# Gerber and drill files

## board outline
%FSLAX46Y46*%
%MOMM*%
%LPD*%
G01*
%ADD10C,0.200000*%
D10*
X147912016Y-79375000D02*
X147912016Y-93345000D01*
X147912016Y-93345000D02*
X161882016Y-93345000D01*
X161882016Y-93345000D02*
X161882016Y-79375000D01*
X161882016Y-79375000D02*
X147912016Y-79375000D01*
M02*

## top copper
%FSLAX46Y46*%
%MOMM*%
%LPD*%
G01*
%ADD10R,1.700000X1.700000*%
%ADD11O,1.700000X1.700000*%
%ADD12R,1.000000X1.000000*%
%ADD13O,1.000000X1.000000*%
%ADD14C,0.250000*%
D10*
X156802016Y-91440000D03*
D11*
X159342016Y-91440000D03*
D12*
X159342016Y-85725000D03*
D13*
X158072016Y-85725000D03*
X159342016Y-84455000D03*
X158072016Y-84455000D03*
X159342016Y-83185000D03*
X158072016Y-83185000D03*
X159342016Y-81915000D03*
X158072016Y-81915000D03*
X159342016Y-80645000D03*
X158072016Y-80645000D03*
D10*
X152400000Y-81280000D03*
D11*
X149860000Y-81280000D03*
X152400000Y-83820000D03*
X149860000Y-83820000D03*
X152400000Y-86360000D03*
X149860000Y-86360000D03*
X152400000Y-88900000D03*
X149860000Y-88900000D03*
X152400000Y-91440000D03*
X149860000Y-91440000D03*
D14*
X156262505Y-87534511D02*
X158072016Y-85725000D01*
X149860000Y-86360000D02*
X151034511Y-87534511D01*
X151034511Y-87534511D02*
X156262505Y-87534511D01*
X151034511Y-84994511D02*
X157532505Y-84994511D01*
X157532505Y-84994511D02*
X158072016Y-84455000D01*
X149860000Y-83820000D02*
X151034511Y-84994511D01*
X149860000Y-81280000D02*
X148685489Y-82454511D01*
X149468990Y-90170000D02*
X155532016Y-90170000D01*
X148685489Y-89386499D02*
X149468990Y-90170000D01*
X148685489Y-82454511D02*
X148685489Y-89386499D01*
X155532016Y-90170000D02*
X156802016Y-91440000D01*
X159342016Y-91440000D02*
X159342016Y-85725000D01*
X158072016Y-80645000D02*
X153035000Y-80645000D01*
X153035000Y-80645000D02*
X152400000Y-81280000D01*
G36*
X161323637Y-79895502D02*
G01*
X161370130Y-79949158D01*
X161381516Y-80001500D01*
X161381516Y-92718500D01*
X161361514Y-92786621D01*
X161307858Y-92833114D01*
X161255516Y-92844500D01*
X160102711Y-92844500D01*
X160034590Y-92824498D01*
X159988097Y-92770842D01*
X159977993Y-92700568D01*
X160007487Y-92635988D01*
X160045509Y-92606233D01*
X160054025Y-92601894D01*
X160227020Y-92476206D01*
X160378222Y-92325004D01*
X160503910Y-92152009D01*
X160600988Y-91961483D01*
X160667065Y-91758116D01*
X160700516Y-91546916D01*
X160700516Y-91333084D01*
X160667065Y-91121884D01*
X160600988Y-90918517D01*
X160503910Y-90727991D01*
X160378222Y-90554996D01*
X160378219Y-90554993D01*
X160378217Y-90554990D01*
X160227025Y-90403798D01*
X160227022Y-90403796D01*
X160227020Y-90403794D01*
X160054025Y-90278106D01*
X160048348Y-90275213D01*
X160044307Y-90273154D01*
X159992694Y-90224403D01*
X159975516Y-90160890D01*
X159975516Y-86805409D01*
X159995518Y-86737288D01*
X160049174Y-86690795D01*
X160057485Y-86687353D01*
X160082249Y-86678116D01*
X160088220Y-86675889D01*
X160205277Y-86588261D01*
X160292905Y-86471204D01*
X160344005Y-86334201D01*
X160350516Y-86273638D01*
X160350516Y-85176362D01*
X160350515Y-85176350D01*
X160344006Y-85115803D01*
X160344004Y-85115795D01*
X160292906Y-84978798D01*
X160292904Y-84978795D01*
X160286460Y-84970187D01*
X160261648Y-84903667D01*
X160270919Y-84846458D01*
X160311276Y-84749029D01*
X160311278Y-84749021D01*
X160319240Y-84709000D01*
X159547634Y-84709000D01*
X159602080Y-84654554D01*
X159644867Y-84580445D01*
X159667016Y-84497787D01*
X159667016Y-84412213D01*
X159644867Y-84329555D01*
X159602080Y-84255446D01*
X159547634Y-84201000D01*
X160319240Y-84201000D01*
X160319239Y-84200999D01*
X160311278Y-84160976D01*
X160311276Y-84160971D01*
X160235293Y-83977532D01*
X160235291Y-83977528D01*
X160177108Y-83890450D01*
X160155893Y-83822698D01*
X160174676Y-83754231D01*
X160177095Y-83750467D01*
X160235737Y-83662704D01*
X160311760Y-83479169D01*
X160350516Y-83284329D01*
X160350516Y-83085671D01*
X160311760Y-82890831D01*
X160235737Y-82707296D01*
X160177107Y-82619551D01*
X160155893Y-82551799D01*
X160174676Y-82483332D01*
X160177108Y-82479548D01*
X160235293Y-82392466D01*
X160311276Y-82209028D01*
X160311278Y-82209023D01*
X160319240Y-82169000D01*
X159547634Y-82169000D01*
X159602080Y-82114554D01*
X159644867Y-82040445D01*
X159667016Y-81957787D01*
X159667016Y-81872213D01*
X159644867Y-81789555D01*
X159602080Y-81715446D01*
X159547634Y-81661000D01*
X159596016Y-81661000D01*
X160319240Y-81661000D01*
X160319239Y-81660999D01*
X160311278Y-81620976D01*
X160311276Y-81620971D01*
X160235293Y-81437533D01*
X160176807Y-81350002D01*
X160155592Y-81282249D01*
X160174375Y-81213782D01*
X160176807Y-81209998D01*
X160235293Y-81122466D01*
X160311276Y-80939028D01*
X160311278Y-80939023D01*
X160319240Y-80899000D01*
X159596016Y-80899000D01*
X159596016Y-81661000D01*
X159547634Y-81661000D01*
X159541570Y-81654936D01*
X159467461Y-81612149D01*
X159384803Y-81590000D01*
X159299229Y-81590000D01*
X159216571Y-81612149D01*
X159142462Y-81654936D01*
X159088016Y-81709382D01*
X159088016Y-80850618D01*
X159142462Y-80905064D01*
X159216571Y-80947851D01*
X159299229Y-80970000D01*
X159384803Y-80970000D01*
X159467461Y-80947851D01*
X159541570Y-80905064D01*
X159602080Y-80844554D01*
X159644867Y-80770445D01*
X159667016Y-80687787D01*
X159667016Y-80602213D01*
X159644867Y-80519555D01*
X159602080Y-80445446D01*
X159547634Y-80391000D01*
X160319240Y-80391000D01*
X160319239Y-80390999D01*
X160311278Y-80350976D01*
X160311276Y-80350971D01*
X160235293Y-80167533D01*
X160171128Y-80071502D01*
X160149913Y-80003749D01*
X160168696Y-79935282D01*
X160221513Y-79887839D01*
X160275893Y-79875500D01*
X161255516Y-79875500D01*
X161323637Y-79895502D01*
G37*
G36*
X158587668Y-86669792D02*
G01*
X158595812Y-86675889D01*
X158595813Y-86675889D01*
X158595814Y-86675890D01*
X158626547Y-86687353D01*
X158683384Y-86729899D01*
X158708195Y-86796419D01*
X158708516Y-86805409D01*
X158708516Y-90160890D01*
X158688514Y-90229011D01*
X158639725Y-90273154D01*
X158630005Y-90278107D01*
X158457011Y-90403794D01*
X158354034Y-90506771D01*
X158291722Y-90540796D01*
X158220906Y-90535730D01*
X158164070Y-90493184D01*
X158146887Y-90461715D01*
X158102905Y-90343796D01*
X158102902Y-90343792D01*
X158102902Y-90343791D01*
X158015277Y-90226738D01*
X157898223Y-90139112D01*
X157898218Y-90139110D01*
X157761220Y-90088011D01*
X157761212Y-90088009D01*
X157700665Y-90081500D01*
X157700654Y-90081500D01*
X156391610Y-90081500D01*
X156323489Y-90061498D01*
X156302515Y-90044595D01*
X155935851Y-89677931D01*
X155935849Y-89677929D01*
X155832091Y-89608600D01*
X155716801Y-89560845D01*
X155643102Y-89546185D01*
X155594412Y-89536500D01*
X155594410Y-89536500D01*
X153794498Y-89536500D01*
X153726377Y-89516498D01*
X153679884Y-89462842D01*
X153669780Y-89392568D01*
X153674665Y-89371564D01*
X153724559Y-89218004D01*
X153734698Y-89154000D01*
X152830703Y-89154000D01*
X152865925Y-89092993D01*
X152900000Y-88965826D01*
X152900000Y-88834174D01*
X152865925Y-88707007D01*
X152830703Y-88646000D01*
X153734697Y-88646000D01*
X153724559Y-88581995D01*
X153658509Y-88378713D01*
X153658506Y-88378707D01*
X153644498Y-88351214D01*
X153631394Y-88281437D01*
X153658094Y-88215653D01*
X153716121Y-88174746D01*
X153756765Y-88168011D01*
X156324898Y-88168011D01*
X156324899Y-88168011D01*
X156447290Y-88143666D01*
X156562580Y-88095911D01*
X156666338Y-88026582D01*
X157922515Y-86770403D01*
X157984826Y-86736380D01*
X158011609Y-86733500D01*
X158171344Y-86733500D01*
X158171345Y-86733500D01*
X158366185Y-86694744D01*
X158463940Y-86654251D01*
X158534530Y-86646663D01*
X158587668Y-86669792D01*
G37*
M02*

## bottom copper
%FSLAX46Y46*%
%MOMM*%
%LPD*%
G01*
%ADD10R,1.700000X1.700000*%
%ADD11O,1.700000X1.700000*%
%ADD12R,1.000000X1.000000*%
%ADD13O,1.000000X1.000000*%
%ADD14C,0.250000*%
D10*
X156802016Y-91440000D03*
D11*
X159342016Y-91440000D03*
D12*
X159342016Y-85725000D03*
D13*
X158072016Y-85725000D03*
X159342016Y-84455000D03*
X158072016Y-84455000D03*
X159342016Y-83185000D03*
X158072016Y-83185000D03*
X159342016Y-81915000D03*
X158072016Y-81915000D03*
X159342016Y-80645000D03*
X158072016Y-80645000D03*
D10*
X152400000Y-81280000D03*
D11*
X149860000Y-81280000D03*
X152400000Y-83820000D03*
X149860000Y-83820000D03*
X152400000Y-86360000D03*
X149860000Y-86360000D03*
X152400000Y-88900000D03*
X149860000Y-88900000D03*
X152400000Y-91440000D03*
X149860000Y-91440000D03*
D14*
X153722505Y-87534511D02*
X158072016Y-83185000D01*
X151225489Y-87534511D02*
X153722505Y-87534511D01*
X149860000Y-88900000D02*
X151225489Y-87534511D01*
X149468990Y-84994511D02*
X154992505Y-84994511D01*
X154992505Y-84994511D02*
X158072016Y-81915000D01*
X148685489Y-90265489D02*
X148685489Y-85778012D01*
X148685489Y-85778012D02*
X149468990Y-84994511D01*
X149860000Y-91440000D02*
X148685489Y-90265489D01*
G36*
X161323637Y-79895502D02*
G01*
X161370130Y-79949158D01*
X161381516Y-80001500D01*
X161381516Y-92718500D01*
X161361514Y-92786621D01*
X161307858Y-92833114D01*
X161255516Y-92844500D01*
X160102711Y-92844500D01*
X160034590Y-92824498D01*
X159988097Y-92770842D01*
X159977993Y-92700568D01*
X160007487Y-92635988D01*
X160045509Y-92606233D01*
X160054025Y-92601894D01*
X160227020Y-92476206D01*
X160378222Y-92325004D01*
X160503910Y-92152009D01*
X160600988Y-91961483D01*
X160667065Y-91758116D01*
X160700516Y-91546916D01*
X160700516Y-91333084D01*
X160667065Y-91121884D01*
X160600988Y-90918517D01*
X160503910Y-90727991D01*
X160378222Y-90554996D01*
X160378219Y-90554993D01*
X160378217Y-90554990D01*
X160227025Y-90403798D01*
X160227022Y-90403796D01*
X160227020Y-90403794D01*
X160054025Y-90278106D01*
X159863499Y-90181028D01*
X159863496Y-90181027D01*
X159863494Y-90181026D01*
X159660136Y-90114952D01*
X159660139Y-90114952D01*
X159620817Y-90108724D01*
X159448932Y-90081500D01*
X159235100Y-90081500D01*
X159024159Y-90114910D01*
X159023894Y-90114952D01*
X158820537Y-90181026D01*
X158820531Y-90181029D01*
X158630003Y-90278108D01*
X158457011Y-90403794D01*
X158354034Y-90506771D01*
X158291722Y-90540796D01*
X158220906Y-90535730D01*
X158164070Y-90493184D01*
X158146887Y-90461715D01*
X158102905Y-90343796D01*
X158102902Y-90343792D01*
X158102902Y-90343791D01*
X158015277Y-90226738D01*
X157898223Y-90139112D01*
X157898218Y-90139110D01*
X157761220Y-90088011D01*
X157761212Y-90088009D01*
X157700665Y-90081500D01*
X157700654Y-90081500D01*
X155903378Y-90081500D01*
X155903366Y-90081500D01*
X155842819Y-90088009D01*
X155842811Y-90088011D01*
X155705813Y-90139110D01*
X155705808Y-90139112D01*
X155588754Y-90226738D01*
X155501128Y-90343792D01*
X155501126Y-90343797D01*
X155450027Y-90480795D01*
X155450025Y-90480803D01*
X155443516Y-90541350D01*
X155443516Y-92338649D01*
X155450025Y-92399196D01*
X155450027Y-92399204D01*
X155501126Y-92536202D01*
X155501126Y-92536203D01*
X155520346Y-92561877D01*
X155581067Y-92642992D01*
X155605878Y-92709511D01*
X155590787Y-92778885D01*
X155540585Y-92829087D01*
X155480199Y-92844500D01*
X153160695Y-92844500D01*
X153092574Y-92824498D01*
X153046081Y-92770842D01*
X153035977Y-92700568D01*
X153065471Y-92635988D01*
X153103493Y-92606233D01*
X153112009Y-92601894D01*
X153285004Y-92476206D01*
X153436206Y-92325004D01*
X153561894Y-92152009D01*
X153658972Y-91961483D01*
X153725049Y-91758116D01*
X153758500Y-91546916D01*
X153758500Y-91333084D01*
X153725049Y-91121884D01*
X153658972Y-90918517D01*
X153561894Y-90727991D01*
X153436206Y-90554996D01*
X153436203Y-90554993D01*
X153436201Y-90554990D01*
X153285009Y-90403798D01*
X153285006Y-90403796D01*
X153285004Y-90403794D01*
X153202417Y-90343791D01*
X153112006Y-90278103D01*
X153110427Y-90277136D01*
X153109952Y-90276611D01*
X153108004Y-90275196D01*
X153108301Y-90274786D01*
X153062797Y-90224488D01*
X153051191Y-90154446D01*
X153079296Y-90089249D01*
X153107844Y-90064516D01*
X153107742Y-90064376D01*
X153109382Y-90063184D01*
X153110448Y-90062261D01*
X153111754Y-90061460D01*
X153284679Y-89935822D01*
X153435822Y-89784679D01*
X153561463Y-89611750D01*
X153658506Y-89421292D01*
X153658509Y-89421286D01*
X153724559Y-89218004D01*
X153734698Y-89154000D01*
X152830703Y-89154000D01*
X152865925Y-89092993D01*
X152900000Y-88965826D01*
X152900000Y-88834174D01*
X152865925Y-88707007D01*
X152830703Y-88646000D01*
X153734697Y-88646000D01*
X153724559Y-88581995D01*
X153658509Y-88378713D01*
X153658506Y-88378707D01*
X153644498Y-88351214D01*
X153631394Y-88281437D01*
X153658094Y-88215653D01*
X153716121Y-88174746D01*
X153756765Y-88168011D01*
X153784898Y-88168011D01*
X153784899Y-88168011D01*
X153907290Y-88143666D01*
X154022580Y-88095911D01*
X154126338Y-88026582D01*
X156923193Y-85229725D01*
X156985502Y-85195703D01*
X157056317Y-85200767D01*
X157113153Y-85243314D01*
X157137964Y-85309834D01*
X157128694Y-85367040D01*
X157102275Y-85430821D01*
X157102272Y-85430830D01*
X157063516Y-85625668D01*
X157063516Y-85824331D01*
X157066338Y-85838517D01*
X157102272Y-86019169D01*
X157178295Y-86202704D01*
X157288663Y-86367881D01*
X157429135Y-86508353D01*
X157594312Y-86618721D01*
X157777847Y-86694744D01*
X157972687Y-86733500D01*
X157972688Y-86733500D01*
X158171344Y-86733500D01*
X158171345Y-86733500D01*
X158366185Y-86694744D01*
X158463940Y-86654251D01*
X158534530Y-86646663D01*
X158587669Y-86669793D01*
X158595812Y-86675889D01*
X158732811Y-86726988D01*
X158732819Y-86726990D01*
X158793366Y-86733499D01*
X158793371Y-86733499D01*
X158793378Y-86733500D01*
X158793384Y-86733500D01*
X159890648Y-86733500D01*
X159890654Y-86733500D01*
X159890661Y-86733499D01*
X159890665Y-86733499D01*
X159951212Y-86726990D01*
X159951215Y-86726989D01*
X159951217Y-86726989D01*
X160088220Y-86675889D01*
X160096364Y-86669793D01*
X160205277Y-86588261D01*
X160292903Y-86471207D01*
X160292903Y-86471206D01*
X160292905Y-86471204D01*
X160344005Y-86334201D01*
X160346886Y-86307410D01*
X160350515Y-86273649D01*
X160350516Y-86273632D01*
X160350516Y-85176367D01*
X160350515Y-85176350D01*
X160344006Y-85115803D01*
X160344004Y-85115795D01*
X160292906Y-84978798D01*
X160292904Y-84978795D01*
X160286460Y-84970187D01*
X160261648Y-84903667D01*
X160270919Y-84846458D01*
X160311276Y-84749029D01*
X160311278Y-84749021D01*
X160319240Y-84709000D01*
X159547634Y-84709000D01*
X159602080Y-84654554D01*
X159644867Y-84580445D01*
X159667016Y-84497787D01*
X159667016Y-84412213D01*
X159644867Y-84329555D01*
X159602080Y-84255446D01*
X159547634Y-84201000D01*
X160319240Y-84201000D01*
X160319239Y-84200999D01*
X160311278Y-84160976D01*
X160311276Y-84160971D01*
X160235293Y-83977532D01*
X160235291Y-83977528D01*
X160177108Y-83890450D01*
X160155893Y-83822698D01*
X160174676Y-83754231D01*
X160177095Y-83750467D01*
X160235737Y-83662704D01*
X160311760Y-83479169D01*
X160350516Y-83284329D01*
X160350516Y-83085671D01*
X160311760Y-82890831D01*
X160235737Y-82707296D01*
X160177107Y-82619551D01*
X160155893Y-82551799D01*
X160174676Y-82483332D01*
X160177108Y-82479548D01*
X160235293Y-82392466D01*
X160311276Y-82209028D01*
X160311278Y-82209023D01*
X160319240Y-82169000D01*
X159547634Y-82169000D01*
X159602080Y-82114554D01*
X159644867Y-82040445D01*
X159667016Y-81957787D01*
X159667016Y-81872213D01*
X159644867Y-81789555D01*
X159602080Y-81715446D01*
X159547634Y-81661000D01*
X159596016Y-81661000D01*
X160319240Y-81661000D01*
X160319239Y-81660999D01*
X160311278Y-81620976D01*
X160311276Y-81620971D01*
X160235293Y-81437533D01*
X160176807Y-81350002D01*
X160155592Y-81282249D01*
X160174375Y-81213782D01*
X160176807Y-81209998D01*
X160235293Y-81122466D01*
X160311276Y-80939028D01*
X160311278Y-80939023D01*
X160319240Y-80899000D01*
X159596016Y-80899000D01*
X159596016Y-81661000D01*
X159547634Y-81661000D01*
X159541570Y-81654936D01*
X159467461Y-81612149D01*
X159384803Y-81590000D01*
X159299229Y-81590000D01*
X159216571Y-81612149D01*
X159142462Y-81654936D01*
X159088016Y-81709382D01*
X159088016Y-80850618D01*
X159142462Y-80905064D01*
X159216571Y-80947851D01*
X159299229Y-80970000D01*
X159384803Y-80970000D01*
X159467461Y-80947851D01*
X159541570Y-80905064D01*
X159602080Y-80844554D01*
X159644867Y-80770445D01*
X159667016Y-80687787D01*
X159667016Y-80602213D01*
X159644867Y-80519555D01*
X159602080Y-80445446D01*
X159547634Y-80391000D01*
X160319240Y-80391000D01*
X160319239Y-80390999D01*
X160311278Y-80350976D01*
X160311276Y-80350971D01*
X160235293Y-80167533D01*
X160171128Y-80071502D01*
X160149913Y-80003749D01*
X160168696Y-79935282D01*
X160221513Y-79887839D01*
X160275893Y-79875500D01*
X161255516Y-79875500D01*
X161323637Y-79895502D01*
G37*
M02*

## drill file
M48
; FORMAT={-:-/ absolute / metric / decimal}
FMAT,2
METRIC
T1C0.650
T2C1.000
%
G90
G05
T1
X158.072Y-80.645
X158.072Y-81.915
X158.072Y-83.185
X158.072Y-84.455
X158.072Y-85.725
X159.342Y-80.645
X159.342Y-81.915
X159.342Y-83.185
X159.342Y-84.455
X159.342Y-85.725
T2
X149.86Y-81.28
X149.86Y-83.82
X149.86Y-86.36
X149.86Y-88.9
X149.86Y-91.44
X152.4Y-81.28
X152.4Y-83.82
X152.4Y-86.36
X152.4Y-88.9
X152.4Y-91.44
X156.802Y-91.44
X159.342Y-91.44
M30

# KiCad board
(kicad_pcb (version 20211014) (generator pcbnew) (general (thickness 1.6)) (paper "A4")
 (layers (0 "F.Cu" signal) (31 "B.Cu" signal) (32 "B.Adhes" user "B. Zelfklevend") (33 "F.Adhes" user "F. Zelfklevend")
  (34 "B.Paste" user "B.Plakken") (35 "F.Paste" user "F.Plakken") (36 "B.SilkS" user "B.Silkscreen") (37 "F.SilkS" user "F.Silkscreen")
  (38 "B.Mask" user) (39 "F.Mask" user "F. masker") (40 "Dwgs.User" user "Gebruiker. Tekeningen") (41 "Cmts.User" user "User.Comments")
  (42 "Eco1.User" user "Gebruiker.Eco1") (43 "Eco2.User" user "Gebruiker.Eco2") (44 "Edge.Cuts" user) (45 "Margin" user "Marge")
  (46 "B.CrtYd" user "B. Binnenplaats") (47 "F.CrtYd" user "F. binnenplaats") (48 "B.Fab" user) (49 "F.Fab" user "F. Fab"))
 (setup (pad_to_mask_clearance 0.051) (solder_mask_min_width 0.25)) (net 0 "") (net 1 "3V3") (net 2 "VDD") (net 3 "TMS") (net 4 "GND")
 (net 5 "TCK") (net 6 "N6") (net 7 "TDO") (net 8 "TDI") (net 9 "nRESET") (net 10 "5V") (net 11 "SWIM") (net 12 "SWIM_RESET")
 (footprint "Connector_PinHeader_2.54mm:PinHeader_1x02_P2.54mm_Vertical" (layer "F.Cu") (at 156.802016 91.44 90)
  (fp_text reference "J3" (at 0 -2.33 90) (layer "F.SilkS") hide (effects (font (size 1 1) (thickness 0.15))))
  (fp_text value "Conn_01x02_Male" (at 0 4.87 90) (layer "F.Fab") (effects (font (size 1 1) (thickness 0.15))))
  (pad "1" thru_hole rect locked (at 0 0 90) (size 1.7 1.7) (drill 1) (layers *.Cu *.Mask) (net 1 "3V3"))
  (pad "2" thru_hole oval locked (at 0 2.54 90) (size 1.7 1.7) (drill 1) (layers *.Cu *.Mask) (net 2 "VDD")))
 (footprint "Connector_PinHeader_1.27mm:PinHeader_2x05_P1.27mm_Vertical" (layer "F.Cu") (at 159.342016 85.725 180)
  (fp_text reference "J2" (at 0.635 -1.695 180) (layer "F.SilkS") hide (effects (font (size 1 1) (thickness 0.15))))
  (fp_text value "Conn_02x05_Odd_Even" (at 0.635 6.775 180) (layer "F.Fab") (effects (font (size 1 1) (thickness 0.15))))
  (pad "1" thru_hole rect locked (at 0 0 180) (size 1 1) (drill 0.65) (layers *.Cu *.Mask) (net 2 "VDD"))
  (pad "2" thru_hole oval locked (at 1.27 0 180) (size 1 1) (drill 0.65) (layers *.Cu *.Mask) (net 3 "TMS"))
  (pad "3" thru_hole oval locked (at 0 1.27 180) (size 1 1) (drill 0.65) (layers *.Cu *.Mask) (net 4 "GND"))
  (pad "4" thru_hole oval locked (at 1.27 1.27 180) (size 1 1) (drill 0.65) (layers *.Cu *.Mask) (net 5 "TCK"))
  (pad "5" thru_hole oval locked (at 0 2.54 180) (size 1 1) (drill 0.65) (layers *.Cu *.Mask) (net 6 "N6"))
  (pad "6" thru_hole oval locked (at 1.27 2.54 180) (size 1 1) (drill 0.65) (layers *.Cu *.Mask) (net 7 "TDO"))
  (pad "7" thru_hole oval locked (at 0 3.81 180) (size 1 1) (drill 0.65) (layers *.Cu *.Mask) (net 4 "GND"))
  (pad "8" thru_hole oval locked (at 1.27 3.81 180) (size 1 1) (drill 0.65) (layers *.Cu *.Mask) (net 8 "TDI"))
  (pad "9" thru_hole oval locked (at 0 5.08 180) (size 1 1) (drill 0.65) (layers *.Cu *.Mask) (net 4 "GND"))
  (pad "10" thru_hole oval locked (at 1.27 5.08 180) (size 1 1) (drill 0.65) (layers *.Cu *.Mask) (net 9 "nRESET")))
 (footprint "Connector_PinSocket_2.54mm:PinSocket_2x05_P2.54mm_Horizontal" (layer "F.Cu") (at 152.4 81.28)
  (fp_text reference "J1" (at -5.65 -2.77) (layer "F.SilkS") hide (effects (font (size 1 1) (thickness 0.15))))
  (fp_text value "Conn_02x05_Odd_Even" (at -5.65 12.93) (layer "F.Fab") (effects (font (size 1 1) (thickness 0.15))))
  (pad "1" thru_hole rect locked (at 0 0) (size 1.7 1.7) (drill 1) (layers *.Cu *.Mask) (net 9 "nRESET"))
  (pad "2" thru_hole oval locked (at -2.54 0) (size 1.7 1.7) (drill 1) (layers *.Cu *.Mask) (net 1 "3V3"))
  (pad "3" thru_hole oval locked (at 0 2.54) (size 1.7 1.7) (drill 1) (layers *.Cu *.Mask) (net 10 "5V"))
  (pad "4" thru_hole oval locked (at -2.54 2.54) (size 1.7 1.7) (drill 1) (layers *.Cu *.Mask) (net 5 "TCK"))
  (pad "5" thru_hole oval locked (at 0 5.08) (size 1.7 1.7) (drill 1) (layers *.Cu *.Mask) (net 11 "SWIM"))
  (pad "6" thru_hole oval locked (at -2.54 5.08) (size 1.7 1.7) (drill 1) (layers *.Cu *.Mask) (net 3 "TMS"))
  (pad "7" thru_hole oval locked (at 0 7.62) (size 1.7 1.7) (drill 1) (layers *.Cu *.Mask) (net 4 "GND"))
  (pad "8" thru_hole oval locked (at -2.54 7.62) (size 1.7 1.7) (drill 1) (layers *.Cu *.Mask) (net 7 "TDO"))
  (pad "9" thru_hole oval locked (at 0 10.16) (size 1.7 1.7) (drill 1) (layers *.Cu *.Mask) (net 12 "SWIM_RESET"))
  (pad "10" thru_hole oval locked (at -2.54 10.16) (size 1.7 1.7) (drill 1) (layers *.Cu *.Mask) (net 8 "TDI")))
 (gr_line (start 147.912016 79.375) (end 147.912016 93.345) (layer "Edge.Cuts") (width 0.2))
 (gr_line (start 147.912016 93.345) (end 161.882016 93.345) (layer "Edge.Cuts") (width 0.2))
 (gr_line (start 161.882016 93.345) (end 161.882016 79.375) (layer "Edge.Cuts") (width 0.2))
 (gr_line (start 161.882016 79.375) (end 147.912016 79.375) (layer "Edge.Cuts") (width 0.2))
 (segment (start 156.262505 87.534511) (end 158.072016 85.725) (width 0.25) (layer "F.Cu") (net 3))
 (segment (start 149.86 86.36) (end 151.034511 87.534511) (width 0.25) (layer "F.Cu") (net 3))
 (segment (start 151.034511 87.534511) (end 156.262505 87.534511) (width 0.25) (layer "F.Cu") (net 3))
 (segment (start 151.034511 84.994511) (end 157.532505 84.994511) (width 0.25) (layer "F.Cu") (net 5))
 (segment (start 157.532505 84.994511) (end 158.072016 84.455) (width 0.25) (layer "F.Cu") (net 5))
 (segment (start 149.86 83.82) (end 151.034511 84.994511) (width 0.25) (layer "F.Cu") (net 5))
 (segment (start 149.86 81.28) (end 148.685489 82.454511) (width 0.25) (layer "F.Cu") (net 1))
 (segment (start 149.46899 90.17) (end 155.532016 90.17) (width 0.25) (layer "F.Cu") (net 1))
 (segment (start 148.685489 89.386499) (end 149.46899 90.17) (width 0.25) (layer "F.Cu") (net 1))
 (segment (start 148.685489 82.454511) (end 148.685489 89.386499) (width 0.25) (layer "F.Cu") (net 1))
 (segment (start 155.532016 90.17) (end 156.802016 91.44) (width 0.25) (layer "F.Cu") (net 1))
 (segment (start 159.342016 91.44) (end 159.342016 85.725) (width 0.25) (layer "F.Cu") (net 2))
 (segment (start 158.072016 80.645) (end 153.035 80.645) (width 0.25) (layer "F.Cu") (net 9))
 (segment (start 153.035 80.645) (end 152.4 81.28) (width 0.25) (layer "F.Cu") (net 9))
 (segment (start 153.722505 87.534511) (end 158.072016 83.185) (width 0.25) (layer "B.Cu") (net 7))
 (segment (start 151.225489 87.534511) (end 153.722505 87.534511) (width 0.25) (layer "B.Cu") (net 7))
 (segment (start 149.86 88.9) (end 151.225489 87.534511) (width 0.25) (layer "B.Cu") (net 7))
 (segment (start 149.46899 84.994511) (end 154.992505 84.994511) (width 0.25) (layer "B.Cu") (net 8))
 (segment (start 154.992505 84.994511) (end 158.072016 81.915) (width 0.25) (layer "B.Cu") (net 8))
 (segment (start 148.685489 90.265489) (end 148.685489 85.778012) (width 0.25) (layer "B.Cu") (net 8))
 (segment (start 148.685489 85.778012) (end 149.46899 84.994511) (width 0.25) (layer "B.Cu") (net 8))
 (segment (start 149.86 91.44) (end 148.685489 90.265489) (width 0.25) (layer "B.Cu") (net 8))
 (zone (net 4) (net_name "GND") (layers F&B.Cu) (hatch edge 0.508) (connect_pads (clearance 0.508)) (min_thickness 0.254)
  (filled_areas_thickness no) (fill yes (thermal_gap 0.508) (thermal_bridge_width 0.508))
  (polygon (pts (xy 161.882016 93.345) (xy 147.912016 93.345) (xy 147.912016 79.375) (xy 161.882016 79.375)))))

